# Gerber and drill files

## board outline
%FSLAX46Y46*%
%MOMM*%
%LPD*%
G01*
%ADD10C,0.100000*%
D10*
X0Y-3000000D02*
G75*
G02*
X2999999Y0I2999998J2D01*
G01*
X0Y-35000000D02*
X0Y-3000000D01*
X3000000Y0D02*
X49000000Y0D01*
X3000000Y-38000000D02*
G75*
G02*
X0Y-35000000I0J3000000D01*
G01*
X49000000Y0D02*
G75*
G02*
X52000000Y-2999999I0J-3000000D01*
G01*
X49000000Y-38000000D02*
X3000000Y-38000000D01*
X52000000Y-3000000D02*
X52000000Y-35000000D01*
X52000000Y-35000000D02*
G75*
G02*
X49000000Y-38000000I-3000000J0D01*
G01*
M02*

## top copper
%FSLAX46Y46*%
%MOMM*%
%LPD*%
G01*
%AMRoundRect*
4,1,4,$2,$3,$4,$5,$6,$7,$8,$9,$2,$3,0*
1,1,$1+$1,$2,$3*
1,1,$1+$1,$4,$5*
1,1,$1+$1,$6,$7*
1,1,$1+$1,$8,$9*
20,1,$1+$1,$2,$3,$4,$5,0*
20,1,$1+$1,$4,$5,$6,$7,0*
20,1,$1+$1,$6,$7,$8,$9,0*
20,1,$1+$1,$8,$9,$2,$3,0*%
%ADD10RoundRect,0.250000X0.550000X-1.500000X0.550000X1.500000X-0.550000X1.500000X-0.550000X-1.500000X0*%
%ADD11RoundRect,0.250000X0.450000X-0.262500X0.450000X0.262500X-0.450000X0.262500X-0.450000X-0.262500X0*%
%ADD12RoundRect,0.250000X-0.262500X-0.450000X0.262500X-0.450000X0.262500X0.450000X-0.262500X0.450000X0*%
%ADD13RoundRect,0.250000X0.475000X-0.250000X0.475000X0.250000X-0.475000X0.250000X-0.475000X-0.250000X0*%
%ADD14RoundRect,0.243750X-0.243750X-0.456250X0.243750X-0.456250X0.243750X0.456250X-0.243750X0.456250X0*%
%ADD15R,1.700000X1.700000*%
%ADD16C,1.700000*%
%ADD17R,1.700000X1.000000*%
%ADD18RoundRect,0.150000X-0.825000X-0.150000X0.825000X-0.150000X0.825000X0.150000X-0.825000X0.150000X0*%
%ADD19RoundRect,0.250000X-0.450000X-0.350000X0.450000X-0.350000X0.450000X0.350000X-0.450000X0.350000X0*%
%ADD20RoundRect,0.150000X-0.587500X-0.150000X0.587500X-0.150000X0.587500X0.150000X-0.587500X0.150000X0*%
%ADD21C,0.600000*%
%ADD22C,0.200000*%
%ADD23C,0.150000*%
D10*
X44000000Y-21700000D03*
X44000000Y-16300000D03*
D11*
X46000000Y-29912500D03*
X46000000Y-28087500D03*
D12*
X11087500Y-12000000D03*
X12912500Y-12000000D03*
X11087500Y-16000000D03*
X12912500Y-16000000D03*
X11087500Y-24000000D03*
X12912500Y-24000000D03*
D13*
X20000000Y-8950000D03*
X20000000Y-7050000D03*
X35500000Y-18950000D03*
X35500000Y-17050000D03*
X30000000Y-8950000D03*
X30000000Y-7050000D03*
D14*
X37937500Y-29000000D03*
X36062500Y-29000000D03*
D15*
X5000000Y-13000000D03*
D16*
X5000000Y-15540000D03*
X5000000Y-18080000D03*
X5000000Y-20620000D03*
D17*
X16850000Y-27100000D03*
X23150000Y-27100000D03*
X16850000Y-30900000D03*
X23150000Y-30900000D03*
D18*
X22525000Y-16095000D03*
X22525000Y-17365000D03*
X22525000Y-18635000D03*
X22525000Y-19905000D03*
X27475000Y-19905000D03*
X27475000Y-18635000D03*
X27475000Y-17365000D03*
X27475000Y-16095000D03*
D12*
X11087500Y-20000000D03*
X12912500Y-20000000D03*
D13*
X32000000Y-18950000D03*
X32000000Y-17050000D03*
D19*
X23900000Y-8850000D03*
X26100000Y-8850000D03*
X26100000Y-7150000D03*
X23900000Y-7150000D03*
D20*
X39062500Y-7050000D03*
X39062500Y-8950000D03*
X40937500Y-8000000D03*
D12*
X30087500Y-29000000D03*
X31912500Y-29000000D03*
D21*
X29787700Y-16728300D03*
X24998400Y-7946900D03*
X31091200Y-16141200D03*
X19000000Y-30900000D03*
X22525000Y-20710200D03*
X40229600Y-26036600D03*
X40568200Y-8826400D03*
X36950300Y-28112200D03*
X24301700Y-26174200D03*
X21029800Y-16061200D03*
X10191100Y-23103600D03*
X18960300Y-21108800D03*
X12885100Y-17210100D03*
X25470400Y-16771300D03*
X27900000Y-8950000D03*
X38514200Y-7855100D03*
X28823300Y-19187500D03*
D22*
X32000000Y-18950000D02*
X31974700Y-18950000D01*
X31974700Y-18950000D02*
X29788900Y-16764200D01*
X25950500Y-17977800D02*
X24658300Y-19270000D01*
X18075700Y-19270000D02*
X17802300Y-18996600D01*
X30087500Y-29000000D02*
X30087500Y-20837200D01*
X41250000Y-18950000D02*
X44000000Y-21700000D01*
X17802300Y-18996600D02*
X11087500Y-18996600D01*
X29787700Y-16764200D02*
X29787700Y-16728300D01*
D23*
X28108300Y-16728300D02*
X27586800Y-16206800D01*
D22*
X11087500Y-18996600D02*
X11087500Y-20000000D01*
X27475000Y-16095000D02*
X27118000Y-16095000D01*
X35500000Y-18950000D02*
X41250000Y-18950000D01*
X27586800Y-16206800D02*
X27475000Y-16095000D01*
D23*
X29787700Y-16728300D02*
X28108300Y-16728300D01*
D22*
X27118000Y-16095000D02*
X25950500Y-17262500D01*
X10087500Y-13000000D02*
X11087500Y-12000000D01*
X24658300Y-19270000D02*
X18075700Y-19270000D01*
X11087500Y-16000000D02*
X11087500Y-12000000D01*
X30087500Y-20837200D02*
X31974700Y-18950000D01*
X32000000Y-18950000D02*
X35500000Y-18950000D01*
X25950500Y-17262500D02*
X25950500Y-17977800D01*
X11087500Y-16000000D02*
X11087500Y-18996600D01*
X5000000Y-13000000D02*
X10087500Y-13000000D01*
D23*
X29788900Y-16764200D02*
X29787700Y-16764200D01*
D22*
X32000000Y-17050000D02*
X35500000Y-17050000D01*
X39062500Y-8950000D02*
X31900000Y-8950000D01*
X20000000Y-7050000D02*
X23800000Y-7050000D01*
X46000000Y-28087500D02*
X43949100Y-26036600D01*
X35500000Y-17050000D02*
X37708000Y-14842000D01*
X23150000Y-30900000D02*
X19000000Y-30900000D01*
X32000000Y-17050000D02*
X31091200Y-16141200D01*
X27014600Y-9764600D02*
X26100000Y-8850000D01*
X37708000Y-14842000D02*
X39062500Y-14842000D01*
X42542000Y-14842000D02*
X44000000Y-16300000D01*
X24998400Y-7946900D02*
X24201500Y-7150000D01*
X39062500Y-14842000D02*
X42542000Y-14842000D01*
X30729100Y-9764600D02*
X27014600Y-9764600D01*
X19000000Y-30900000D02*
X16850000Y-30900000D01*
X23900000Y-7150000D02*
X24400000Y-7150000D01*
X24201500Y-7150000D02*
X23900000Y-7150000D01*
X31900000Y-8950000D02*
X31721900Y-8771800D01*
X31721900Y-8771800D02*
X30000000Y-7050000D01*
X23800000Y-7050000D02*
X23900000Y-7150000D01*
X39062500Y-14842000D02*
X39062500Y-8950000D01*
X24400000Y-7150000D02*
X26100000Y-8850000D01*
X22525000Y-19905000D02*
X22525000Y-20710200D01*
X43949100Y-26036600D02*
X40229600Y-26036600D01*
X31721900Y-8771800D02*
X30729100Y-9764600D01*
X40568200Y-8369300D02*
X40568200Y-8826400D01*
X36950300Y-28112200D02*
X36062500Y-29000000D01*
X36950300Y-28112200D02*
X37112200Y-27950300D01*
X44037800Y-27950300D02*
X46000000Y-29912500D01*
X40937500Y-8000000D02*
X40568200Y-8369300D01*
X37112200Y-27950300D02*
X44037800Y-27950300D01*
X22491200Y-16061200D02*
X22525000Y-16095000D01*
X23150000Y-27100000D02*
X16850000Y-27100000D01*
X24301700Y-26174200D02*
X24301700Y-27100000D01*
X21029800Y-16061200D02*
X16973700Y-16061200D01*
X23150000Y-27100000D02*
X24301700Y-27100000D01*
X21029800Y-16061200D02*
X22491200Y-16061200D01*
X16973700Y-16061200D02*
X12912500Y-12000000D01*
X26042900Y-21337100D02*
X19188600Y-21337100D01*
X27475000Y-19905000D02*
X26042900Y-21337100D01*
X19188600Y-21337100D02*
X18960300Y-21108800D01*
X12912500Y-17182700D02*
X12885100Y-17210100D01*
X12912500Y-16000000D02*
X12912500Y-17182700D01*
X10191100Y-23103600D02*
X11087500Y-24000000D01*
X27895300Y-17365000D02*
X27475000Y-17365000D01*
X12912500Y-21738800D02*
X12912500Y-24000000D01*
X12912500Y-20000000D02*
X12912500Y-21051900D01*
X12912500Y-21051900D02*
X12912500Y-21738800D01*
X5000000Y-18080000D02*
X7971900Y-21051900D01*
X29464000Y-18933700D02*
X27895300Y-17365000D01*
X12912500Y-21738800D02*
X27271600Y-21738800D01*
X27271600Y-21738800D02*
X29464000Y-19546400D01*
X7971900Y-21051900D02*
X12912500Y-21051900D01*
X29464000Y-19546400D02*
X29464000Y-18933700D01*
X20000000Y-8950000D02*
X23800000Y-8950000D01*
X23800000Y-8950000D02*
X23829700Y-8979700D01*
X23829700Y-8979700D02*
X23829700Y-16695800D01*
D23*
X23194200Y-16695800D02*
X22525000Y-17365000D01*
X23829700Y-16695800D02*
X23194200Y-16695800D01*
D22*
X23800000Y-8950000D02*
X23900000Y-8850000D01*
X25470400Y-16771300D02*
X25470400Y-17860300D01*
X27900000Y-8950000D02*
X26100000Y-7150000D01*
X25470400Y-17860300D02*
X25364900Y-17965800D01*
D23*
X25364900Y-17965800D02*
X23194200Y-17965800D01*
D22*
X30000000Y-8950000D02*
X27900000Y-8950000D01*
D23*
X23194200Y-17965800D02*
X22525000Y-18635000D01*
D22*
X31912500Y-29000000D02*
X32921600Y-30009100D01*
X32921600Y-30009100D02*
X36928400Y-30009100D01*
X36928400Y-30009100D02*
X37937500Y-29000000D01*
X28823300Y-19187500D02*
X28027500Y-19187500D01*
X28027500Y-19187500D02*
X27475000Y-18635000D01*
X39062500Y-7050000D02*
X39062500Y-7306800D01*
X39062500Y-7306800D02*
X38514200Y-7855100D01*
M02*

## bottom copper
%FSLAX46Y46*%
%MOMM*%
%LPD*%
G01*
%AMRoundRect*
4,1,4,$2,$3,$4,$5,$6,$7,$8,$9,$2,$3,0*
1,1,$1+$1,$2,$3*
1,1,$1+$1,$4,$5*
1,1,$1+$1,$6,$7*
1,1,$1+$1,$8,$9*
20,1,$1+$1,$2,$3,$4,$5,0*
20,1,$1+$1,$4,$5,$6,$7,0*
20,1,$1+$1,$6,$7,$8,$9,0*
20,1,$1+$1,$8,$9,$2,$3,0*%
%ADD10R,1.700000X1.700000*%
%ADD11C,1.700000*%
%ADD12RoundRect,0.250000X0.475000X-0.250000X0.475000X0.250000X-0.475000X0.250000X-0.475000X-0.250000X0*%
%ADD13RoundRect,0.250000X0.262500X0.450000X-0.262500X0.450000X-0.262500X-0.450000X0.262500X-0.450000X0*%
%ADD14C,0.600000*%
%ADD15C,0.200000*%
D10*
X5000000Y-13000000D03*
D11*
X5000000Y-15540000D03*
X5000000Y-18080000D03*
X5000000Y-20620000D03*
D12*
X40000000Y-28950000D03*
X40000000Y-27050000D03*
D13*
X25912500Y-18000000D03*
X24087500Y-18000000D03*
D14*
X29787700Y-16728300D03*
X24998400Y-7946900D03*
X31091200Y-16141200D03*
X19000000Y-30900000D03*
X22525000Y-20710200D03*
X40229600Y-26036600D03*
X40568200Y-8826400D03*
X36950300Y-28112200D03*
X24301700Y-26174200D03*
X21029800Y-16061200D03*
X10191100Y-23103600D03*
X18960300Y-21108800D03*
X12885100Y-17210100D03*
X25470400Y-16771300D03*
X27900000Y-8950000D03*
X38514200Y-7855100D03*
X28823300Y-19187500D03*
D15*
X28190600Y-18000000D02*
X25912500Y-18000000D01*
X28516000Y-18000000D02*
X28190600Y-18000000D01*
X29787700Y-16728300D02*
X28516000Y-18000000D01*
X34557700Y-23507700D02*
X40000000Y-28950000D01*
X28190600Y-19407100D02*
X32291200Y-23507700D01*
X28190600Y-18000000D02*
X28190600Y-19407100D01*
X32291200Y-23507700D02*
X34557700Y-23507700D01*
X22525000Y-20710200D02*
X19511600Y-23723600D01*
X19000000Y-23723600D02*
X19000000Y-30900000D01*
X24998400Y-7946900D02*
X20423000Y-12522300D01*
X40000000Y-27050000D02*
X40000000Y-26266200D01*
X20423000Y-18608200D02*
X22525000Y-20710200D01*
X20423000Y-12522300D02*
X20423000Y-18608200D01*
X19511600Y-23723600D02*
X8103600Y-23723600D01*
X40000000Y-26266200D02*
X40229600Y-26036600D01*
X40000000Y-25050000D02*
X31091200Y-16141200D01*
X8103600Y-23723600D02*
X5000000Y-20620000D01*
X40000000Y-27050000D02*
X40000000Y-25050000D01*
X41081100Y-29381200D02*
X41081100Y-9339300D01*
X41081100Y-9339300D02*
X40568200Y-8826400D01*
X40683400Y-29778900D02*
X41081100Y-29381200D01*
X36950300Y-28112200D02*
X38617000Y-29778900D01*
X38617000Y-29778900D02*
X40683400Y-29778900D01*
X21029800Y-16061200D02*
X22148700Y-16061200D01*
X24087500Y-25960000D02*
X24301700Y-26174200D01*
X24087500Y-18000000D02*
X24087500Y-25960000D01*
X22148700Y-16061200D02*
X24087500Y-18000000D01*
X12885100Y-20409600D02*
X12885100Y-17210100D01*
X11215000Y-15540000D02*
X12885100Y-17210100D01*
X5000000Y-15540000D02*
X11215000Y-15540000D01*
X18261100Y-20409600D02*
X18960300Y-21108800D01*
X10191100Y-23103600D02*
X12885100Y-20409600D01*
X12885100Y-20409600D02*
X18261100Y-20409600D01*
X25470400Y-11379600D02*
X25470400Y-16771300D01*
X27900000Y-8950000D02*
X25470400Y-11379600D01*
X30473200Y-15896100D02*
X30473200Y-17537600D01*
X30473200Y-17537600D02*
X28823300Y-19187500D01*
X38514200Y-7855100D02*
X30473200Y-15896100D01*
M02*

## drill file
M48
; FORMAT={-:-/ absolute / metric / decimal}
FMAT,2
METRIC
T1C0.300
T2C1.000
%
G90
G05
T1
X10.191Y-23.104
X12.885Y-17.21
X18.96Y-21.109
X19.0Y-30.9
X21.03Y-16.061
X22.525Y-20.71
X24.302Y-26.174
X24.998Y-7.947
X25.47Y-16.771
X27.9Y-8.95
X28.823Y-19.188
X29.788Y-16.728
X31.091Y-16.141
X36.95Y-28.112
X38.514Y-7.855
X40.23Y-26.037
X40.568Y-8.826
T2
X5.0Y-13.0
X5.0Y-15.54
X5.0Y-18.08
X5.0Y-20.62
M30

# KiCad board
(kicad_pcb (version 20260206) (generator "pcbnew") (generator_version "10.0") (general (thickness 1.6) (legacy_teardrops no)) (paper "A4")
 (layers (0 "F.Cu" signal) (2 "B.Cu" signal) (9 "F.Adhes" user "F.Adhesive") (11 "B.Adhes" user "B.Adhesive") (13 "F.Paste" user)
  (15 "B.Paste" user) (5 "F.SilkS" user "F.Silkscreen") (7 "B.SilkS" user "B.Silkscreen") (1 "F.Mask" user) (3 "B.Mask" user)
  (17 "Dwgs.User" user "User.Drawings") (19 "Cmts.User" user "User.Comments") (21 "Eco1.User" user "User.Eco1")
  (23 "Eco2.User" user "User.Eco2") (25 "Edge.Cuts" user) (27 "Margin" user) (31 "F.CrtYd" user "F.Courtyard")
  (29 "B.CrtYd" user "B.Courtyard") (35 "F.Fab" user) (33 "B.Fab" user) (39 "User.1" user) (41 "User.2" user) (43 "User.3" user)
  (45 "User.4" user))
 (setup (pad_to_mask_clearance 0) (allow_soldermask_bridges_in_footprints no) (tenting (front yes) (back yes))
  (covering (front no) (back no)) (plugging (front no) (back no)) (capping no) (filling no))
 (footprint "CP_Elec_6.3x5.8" (layer "F.Cu") (at 44 19 90)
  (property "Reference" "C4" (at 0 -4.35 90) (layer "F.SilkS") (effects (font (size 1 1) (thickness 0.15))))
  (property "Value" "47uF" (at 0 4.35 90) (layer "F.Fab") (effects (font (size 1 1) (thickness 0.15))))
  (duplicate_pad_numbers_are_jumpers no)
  (pad "1" smd roundrect (at -2.7 0 90) (size 3.5 1.6) (layers "F.Cu" "F.Mask" "F.Paste") (roundrect_rratio 0.15625) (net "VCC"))
  (pad "2" smd roundrect (at 2.7 0 90) (size 3.5 1.6) (layers "F.Cu" "F.Mask" "F.Paste") (roundrect_rratio 0.15625) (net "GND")))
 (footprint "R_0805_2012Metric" (layer "F.Cu") (at 46 29 90)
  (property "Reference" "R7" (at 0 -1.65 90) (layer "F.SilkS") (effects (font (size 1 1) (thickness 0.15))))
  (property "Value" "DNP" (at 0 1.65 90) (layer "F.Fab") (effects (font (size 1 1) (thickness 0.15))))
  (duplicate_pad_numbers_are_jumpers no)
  (pad "1" smd roundrect (at -0.9125 0 90) (size 1.025 1.4) (layers "F.Cu" "F.Mask" "F.Paste") (roundrect_rratio 0.243902) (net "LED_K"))
  (pad "2" smd roundrect (at 0.9125 0 90) (size 1.025 1.4) (layers "F.Cu" "F.Mask" "F.Paste") (roundrect_rratio 0.243902) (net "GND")))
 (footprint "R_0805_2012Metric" (layer "F.Cu") (at 12 12)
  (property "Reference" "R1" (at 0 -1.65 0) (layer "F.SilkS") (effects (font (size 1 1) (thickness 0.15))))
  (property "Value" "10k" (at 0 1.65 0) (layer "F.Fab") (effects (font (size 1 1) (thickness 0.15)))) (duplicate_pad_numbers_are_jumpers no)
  (pad "1" smd roundrect (at -0.9125 0) (size 1.025 1.4) (layers "F.Cu" "F.Mask" "F.Paste") (roundrect_rratio 0.243902) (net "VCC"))
  (pad "2" smd roundrect (at 0.9125 0) (size 1.025 1.4) (layers "F.Cu" "F.Mask" "F.Paste") (roundrect_rratio 0.243902) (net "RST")))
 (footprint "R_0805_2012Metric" (layer "F.Cu") (at 12 16)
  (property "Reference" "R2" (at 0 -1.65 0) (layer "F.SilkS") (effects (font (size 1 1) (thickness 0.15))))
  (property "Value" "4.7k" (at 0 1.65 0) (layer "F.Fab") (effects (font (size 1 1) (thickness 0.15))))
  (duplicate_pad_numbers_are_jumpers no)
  (pad "1" smd roundrect (at -0.9125 0) (size 1.025 1.4) (layers "F.Cu" "F.Mask" "F.Paste") (roundrect_rratio 0.243902) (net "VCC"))
  (pad "2" smd roundrect (at 0.9125 0) (size 1.025 1.4) (layers "F.Cu" "F.Mask" "F.Paste") (roundrect_rratio 0.243902) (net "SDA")))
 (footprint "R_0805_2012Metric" (layer "F.Cu") (at 12 24)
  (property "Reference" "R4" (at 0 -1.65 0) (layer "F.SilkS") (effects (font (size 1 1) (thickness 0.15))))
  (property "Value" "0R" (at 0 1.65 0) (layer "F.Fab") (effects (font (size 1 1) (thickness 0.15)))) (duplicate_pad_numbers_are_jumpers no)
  (pad "1" smd roundrect (at -0.9125 0) (size 1.025 1.4) (layers "F.Cu" "F.Mask" "F.Paste") (roundrect_rratio 0.243902) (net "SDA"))
  (pad "2" smd roundrect (at 0.9125 0) (size 1.025 1.4) (layers "F.Cu" "F.Mask" "F.Paste") (roundrect_rratio 0.243902) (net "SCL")))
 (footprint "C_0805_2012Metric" (layer "F.Cu") (at 20 8 90)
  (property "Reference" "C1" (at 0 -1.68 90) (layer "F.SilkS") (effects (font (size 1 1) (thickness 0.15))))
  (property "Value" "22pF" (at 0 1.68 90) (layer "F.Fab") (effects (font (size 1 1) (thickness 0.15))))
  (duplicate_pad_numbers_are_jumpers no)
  (pad "1" smd roundrect (at -0.95 0 90) (size 1 1.45) (layers "F.Cu" "F.Mask" "F.Paste") (roundrect_rratio 0.25) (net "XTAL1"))
  (pad "2" smd roundrect (at 0.95 0 90) (size 1 1.45) (layers "F.Cu" "F.Mask" "F.Paste") (roundrect_rratio 0.25) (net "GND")))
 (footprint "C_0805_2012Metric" (layer "F.Cu") (at 35.5 18 90)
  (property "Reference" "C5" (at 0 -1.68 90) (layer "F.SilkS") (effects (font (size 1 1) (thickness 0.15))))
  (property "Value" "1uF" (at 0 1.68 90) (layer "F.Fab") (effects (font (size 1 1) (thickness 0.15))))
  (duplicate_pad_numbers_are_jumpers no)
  (pad "1" smd roundrect (at -0.95 0 90) (size 1 1.45) (layers "F.Cu" "F.Mask" "F.Paste") (roundrect_rratio 0.25) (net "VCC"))
  (pad "2" smd roundrect (at 0.95 0 90) (size 1 1.45) (layers "F.Cu" "F.Mask" "F.Paste") (roundrect_rratio 0.25) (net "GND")))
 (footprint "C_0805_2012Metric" (layer "F.Cu") (at 30 8 90)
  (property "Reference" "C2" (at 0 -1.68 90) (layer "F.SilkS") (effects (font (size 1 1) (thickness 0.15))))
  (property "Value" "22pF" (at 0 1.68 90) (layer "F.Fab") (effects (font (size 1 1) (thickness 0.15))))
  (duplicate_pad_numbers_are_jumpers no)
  (pad "1" smd roundrect (at -0.95 0 90) (size 1 1.45) (layers "F.Cu" "F.Mask" "F.Paste") (roundrect_rratio 0.25) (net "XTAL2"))
  (pad "2" smd roundrect (at 0.95 0 90) (size 1 1.45) (layers "F.Cu" "F.Mask" "F.Paste") (roundrect_rratio 0.25) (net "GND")))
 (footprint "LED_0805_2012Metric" (layer "F.Cu") (at 37 29)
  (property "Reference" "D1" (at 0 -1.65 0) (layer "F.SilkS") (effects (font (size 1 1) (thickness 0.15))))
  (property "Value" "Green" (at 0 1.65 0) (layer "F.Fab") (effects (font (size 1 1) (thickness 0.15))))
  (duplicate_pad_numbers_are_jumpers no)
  (pad "A" smd roundrect (at 0.9375 0) (size 0.975 1.4) (layers "F.Cu" "F.Mask" "F.Paste") (roundrect_rratio 0.25) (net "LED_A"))
  (pad "K" smd roundrect (at -0.9375 0) (size 0.975 1.4) (layers "F.Cu" "F.Mask" "F.Paste") (roundrect_rratio 0.25) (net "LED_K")))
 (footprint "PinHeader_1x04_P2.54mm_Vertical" (layer "F.Cu") (at 5 13)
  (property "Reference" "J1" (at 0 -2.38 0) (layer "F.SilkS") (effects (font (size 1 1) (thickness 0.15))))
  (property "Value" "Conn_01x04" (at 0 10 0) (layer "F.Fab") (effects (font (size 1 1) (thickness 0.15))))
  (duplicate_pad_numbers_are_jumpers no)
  (pad "1" thru_hole rect (at 0 0) (size 1.7 1.7) (drill 1) (layers "*.Cu" "*.Mask") (remove_unused_layers no) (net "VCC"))
  (pad "2" thru_hole circle (at 0 2.54) (size 1.7 1.7) (drill 1) (layers "*.Cu" "*.Mask") (remove_unused_layers no) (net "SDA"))
  (pad "3" thru_hole circle (at 0 5.08) (size 1.7 1.7) (drill 1) (layers "*.Cu" "*.Mask") (remove_unused_layers no) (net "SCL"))
  (pad "4" thru_hole circle (at 0 7.62) (size 1.7 1.7) (drill 1) (layers "*.Cu" "*.Mask") (remove_unused_layers no) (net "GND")))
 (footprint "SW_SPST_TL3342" (layer "F.Cu") (at 20 29)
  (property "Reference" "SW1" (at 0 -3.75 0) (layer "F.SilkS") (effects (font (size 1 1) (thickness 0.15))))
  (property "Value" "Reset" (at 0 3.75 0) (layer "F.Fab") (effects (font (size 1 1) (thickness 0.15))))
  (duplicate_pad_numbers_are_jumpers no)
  (pad "1" smd rect (at -3.15 -1.9) (size 1.7 1) (layers "F.Cu" "F.Mask" "F.Paste") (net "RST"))
  (pad "1" smd rect (at 3.15 -1.9) (size 1.7 1) (layers "F.Cu" "F.Mask" "F.Paste") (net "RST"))
  (pad "2" smd rect (at -3.15 1.9) (size 1.7 1) (layers "F.Cu" "F.Mask" "F.Paste") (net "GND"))
  (pad "2" smd rect (at 3.15 1.9) (size 1.7 1) (layers "F.Cu" "F.Mask" "F.Paste") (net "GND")))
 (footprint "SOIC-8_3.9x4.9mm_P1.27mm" (layer "F.Cu") (at 25 18)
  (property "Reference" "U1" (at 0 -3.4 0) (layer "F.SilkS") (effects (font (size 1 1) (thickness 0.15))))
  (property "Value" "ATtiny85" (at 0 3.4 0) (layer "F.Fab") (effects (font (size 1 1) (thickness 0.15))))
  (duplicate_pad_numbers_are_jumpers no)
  (pad "1" smd roundrect (at -2.475 -1.905) (size 1.95 0.6) (layers "F.Cu" "F.Mask" "F.Paste") (roundrect_rratio 0.25) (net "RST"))
  (pad "2" smd roundrect (at -2.475 -0.635) (size 1.95 0.6) (layers "F.Cu" "F.Mask" "F.Paste") (roundrect_rratio 0.25) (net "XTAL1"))
  (pad "3" smd roundrect (at -2.475 0.635) (size 1.95 0.6) (layers "F.Cu" "F.Mask" "F.Paste") (roundrect_rratio 0.25) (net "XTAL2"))
  (pad "4" smd roundrect (at -2.475 1.905) (size 1.95 0.6) (layers "F.Cu" "F.Mask" "F.Paste") (roundrect_rratio 0.25) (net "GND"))
  (pad "5" smd roundrect (at 2.475 1.905) (size 1.95 0.6) (layers "F.Cu" "F.Mask" "F.Paste") (roundrect_rratio 0.25) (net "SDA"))
  (pad "6" smd roundrect (at 2.475 0.635) (size 1.95 0.6) (layers "F.Cu" "F.Mask" "F.Paste") (roundrect_rratio 0.25) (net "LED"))
  (pad "7" smd roundrect (at 2.475 -0.635) (size 1.95 0.6) (layers "F.Cu" "F.Mask" "F.Paste") (roundrect_rratio 0.25) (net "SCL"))
  (pad "8" smd roundrect (at 2.475 -1.905) (size 1.95 0.6) (layers "F.Cu" "F.Mask" "F.Paste") (roundrect_rratio 0.25) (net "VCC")))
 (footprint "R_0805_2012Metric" (layer "F.Cu") (at 12 20)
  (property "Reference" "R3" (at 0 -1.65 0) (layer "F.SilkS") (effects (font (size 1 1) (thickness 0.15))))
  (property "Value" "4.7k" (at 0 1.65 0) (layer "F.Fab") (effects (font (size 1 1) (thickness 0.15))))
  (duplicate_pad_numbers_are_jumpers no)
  (pad "1" smd roundrect (at -0.9125 0) (size 1.025 1.4) (layers "F.Cu" "F.Mask" "F.Paste") (roundrect_rratio 0.243902) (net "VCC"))
  (pad "2" smd roundrect (at 0.9125 0) (size 1.025 1.4) (layers "F.Cu" "F.Mask" "F.Paste") (roundrect_rratio 0.243902) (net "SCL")))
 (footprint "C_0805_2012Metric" (layer "F.Cu") (at 32 18 90)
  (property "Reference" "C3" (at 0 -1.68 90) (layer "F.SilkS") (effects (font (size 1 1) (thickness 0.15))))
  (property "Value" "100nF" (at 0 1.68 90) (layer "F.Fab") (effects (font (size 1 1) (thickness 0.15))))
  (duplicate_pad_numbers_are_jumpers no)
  (pad "1" smd roundrect (at -0.95 0 90) (size 1 1.45) (layers "F.Cu" "F.Mask" "F.Paste") (roundrect_rratio 0.25) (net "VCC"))
  (pad "2" smd roundrect (at 0.95 0 90) (size 1 1.45) (layers "F.Cu" "F.Mask" "F.Paste") (roundrect_rratio 0.25) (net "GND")))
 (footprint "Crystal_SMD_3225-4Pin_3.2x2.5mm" (layer "F.Cu") (at 25 8)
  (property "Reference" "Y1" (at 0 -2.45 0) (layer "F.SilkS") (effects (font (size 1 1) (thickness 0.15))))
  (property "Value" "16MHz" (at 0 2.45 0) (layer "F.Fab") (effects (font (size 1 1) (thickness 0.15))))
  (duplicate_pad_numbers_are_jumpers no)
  (pad "1" smd roundrect (at -1.1 0.85) (size 1.4 1.2) (layers "F.Cu" "F.Mask" "F.Paste") (roundrect_rratio 0.208333) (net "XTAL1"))
  (pad "2" smd roundrect (at 1.1 0.85) (size 1.4 1.2) (layers "F.Cu" "F.Mask" "F.Paste") (roundrect_rratio 0.208333) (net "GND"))
  (pad "3" smd roundrect (at 1.1 -0.85) (size 1.4 1.2) (layers "F.Cu" "F.Mask" "F.Paste") (roundrect_rratio 0.208333) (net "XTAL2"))
  (pad "4" smd roundrect (at -1.1 -0.85) (size 1.4 1.2) (layers "F.Cu" "F.Mask" "F.Paste") (roundrect_rratio 0.208333) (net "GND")))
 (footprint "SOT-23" (layer "F.Cu") (at 40 8)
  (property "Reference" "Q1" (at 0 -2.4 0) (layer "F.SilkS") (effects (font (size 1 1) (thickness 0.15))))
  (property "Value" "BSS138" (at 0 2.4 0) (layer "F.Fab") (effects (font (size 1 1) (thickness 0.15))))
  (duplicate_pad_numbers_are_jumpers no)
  (pad "1" smd roundrect (at -0.9375 -0.95) (size 1.475 0.6) (layers "F.Cu" "F.Mask" "F.Paste") (roundrect_rratio 0.25) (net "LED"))
  (pad "2" smd roundrect (at -0.9375 0.95) (size 1.475 0.6) (layers "F.Cu" "F.Mask" "F.Paste") (roundrect_rratio 0.25) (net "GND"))
  (pad "3" smd roundrect (at 0.9375 0) (size 1.475 0.6) (layers "F.Cu" "F.Mask" "F.Paste") (roundrect_rratio 0.25) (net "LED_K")))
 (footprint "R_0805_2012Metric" (layer "F.Cu") (at 31 29)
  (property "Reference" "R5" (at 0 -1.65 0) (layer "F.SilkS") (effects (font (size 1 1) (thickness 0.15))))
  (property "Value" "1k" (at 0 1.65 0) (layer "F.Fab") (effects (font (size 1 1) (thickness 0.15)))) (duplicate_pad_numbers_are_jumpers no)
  (pad "1" smd roundrect (at -0.9125 0) (size 1.025 1.4) (layers "F.Cu" "F.Mask" "F.Paste") (roundrect_rratio 0.243902) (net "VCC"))
  (pad "2" smd roundrect (at 0.9125 0) (size 1.025 1.4) (layers "F.Cu" "F.Mask" "F.Paste") (roundrect_rratio 0.243902) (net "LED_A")))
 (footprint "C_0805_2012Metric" (layer "B.Cu") (at 40 28 90)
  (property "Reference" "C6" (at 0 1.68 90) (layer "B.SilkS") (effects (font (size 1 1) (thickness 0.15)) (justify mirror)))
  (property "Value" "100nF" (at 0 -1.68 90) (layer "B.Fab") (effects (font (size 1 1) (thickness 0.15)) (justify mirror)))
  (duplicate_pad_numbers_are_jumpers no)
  (pad "1" smd roundrect (at -0.95 0 90) (size 1 1.45) (layers "B.Cu" "B.Mask" "B.Paste") (roundrect_rratio 0.25) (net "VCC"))
  (pad "2" smd roundrect (at 0.95 0 90) (size 1 1.45) (layers "B.Cu" "B.Mask" "B.Paste") (roundrect_rratio 0.25) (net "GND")))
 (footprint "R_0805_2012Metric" (layer "B.Cu") (at 25 18 180)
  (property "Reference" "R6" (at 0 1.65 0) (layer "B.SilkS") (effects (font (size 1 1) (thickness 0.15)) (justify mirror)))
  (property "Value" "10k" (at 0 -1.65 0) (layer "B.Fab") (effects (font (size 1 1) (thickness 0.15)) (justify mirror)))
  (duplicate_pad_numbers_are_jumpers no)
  (pad "1" smd roundrect (at -0.9125 0 180) (size 1.025 1.4) (layers "B.Cu" "B.Mask" "B.Paste") (roundrect_rratio 0.243902) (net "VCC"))
  (pad "2" smd roundrect (at 0.9125 0 180) (size 1.025 1.4) (layers "B.Cu" "B.Mask" "B.Paste") (roundrect_rratio 0.243902) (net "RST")))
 (gr_arc (start 0 3) (mid 0.878679 0.878679) (end 2.999999 0) (stroke (width 0.1) (type default)) (layer "Edge.Cuts"))
 (gr_line (start 0 35) (end 0 3) (stroke (width 0.1) (type default)) (layer "Edge.Cuts"))
 (gr_line (start 3 0) (end 49 0) (stroke (width 0.1) (type default)) (layer "Edge.Cuts"))
 (gr_arc (start 3 38) (mid 0.878679 37.12132) (end 0 35) (stroke (width 0.1) (type default)) (layer "Edge.Cuts"))
 (gr_arc (start 49 0) (mid 51.12132 0.878679) (end 52 2.999999) (stroke (width 0.1) (type default)) (layer "Edge.Cuts"))
 (gr_line (start 49 38) (end 3 38) (stroke (width 0.1) (type default)) (layer "Edge.Cuts"))
 (gr_line (start 52 3) (end 52 35) (stroke (width 0.1) (type default)) (layer "Edge.Cuts"))
 (gr_arc (start 52 35) (mid 51.12132 37.12132) (end 49 38) (stroke (width 0.1) (type default)) (layer "Edge.Cuts"))
 (segment (start 32 18.95) (end 31.9747 18.95) (width 0.2) (layer "F.Cu") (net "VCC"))
 (segment (start 31.9747 18.95) (end 29.7889 16.7642) (width 0.2) (layer "F.Cu") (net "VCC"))
 (segment (start 25.9505 17.9778) (end 24.6583 19.27) (width 0.2) (layer "F.Cu") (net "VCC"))
 (segment (start 18.0757 19.27) (end 17.8023 18.9966) (width 0.2) (layer "F.Cu") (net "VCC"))
 (segment (start 30.0875 29) (end 30.0875 20.8372) (width 0.2) (layer "F.Cu") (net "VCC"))
 (segment (start 41.25 18.95) (end 44 21.7) (width 0.2) (layer "F.Cu") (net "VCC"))
 (segment (start 17.8023 18.9966) (end 11.0875 18.9966) (width 0.2) (layer "F.Cu") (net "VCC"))
 (segment (start 29.7877 16.7642) (end 29.7877 16.7283) (width 0.2) (layer "F.Cu") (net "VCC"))
 (segment (start 28.1083 16.7283) (end 27.5868 16.2068) (width 0.15) (layer "F.Cu") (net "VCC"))
 (segment (start 11.0875 18.9966) (end 11.0875 20) (width 0.2) (layer "F.Cu") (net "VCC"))
 (segment (start 27.475 16.095) (end 27.118 16.095) (width 0.2) (layer "F.Cu") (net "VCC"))
 (segment (start 35.5 18.95) (end 41.25 18.95) (width 0.2) (layer "F.Cu") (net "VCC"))
 (segment (start 27.5868 16.2068) (end 27.475 16.095) (width 0.2) (layer "F.Cu") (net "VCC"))
 (segment (start 29.7877 16.7283) (end 28.1083 16.7283) (width 0.15) (layer "F.Cu") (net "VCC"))
 (segment (start 27.118 16.095) (end 25.9505 17.2625) (width 0.2) (layer "F.Cu") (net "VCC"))
 (segment (start 10.0875 13) (end 11.0875 12) (width 0.2) (layer "F.Cu") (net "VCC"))
 (segment (start 24.6583 19.27) (end 18.0757 19.27) (width 0.2) (layer "F.Cu") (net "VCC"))
 (segment (start 11.0875 16) (end 11.0875 12) (width 0.2) (layer "F.Cu") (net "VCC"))
 (segment (start 30.0875 20.8372) (end 31.9747 18.95) (width 0.2) (layer "F.Cu") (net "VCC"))
 (segment (start 32 18.95) (end 35.5 18.95) (width 0.2) (layer "F.Cu") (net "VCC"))
 (segment (start 25.9505 17.2625) (end 25.9505 17.9778) (width 0.2) (layer "F.Cu") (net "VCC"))
 (segment (start 11.0875 16) (end 11.0875 18.9966) (width 0.2) (layer "F.Cu") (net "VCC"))
 (segment (start 5 13) (end 10.0875 13) (width 0.2) (layer "F.Cu") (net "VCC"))
 (segment (start 29.7889 16.7642) (end 29.7877 16.7642) (width 0.15) (layer "F.Cu") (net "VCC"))
 (via (at 29.7877 16.7283) (size 0.6) (drill 0.3) (layers "F.Cu" "B.Cu") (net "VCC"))
 (segment (start 28.1906 18) (end 25.9125 18) (width 0.2) (layer "B.Cu") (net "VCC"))
 (segment (start 28.516 18) (end 28.1906 18) (width 0.2) (layer "B.Cu") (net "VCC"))
 (segment (start 29.7877 16.7283) (end 28.516 18) (width 0.2) (layer "B.Cu") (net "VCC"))
 (segment (start 34.5577 23.5077) (end 40 28.95) (width 0.2) (layer "B.Cu") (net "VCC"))
 (segment (start 28.1906 19.4071) (end 32.2912 23.5077) (width 0.2) (layer "B.Cu") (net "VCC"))
 (segment (start 28.1906 18) (end 28.1906 19.4071) (width 0.2) (layer "B.Cu") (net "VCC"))
 (segment (start 32.2912 23.5077) (end 34.5577 23.5077) (width 0.2) (layer "B.Cu") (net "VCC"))
 (segment (start 32 17.05) (end 35.5 17.05) (width 0.2) (layer "F.Cu") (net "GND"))
 (segment (start 39.0625 8.95) (end 31.9 8.95) (width 0.2) (layer "F.Cu") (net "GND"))
 (segment (start 20 7.05) (end 23.8 7.05) (width 0.2) (layer "F.Cu") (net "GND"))
 (segment (start 46 28.0875) (end 43.9491 26.0366) (width 0.2) (layer "F.Cu") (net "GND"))
 (segment (start 35.5 17.05) (end 37.708 14.842) (width 0.2) (layer "F.Cu") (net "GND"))
 (segment (start 23.15 30.9) (end 19 30.9) (width 0.2) (layer "F.Cu") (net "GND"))
 (segment (start 32 17.05) (end 31.0912 16.1412) (width 0.2) (layer "F.Cu") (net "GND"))
 (segment (start 27.0146 9.7646) (end 26.1 8.85) (width 0.2) (layer "F.Cu") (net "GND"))
 (segment (start 37.708 14.842) (end 39.0625 14.842) (width 0.2) (layer "F.Cu") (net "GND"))
 (segment (start 42.542 14.842) (end 44 16.3) (width 0.2) (layer "F.Cu") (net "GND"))
 (segment (start 24.9984 7.9469) (end 24.2015 7.15) (width 0.2) (layer "F.Cu") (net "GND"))
 (segment (start 39.0625 14.842) (end 42.542 14.842) (width 0.2) (layer "F.Cu") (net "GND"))
 (segment (start 30.7291 9.7646) (end 27.0146 9.7646) (width 0.2) (layer "F.Cu") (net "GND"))
 (segment (start 19 30.9) (end 16.85 30.9) (width 0.2) (layer "F.Cu") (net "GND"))
 (segment (start 23.9 7.15) (end 24.4 7.15) (width 0.2) (layer "F.Cu") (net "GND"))
 (segment (start 24.2015 7.15) (end 23.9 7.15) (width 0.2) (layer "F.Cu") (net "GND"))
 (segment (start 31.9 8.95) (end 31.7219 8.7718) (width 0.2) (layer "F.Cu") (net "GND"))
 (segment (start 31.7219 8.7718) (end 30 7.05) (width 0.2) (layer "F.Cu") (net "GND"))
 (segment (start 23.8 7.05) (end 23.9 7.15) (width 0.2) (layer "F.Cu") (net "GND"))
 (segment (start 39.0625 14.842) (end 39.0625 8.95) (width 0.2) (layer "F.Cu") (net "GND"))
 (segment (start 24.4 7.15) (end 26.1 8.85) (width 0.2) (layer "F.Cu") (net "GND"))
 (segment (start 22.525 19.905) (end 22.525 20.7102) (width 0.2) (layer "F.Cu") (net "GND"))
 (segment (start 43.9491 26.0366) (end 40.2296 26.0366) (width 0.2) (layer "F.Cu") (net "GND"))
 (segment (start 31.7219 8.7718) (end 30.7291 9.7646) (width 0.2) (layer "F.Cu") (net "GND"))
 (via (at 24.9984 7.9469) (size 0.6) (drill 0.3) (layers "F.Cu" "B.Cu") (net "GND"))
 (via (at 31.0912 16.1412) (size 0.6) (drill 0.3) (layers "F.Cu" "B.Cu") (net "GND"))
 (via (at 19 30.9) (size 0.6) (drill 0.3) (layers "F.Cu" "B.Cu") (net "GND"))
 (via (at 22.525 20.7102) (size 0.6) (drill 0.3) (layers "F.Cu" "B.Cu") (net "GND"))
 (via (at 40.2296 26.0366) (size 0.6) (drill 0.3) (layers "F.Cu" "B.Cu") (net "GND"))
 (segment (start 22.525 20.7102) (end 19.5116 23.7236) (width 0.2) (layer "B.Cu") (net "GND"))
 (segment (start 19 23.7236) (end 19 30.9) (width 0.2) (layer "B.Cu") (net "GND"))
 (segment (start 24.9984 7.9469) (end 20.423 12.5223) (width 0.2) (layer "B.Cu") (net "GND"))
 (segment (start 40 27.05) (end 40 26.2662) (width 0.2) (layer "B.Cu") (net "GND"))
 (segment (start 20.423 18.6082) (end 22.525 20.7102) (width 0.2) (layer "B.Cu") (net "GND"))
 (segment (start 20.423 12.5223) (end 20.423 18.6082) (width 0.2) (layer "B.Cu") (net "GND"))
 (segment (start 19.5116 23.7236) (end 8.1036 23.7236) (width 0.2) (layer "B.Cu") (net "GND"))
 (segment (start 40 26.2662) (end 40.2296 26.0366) (width 0.2) (layer "B.Cu") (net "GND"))
 (segment (start 40 25.05) (end 31.0912 16.1412) (width 0.2) (layer "B.Cu") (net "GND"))
 (segment (start 8.1036 23.7236) (end 5 20.62) (width 0.2) (layer "B.Cu") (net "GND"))
 (segment (start 40 27.05) (end 40 25.05) (width 0.2) (layer "B.Cu") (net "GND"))
 (segment (start 40.5682 8.3693) (end 40.5682 8.8264) (width 0.2) (layer "F.Cu") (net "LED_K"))
 (segment (start 36.9503 28.1122) (end 36.0625 29) (width 0.2) (layer "F.Cu") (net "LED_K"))
 (segment (start 36.9503 28.1122) (end 37.1122 27.9503) (width 0.2) (layer "F.Cu") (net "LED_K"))
 (segment (start 44.0378 27.9503) (end 46 29.9125) (width 0.2) (layer "F.Cu") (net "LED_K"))
 (segment (start 40.9375 8) (end 40.5682 8.3693) (width 0.2) (layer "F.Cu") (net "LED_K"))
 (segment (start 37.1122 27.9503) (end 44.0378 27.9503) (width 0.2) (layer "F.Cu") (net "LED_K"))
 (via (at 40.5682 8.8264) (size 0.6) (drill 0.3) (layers "F.Cu" "B.Cu") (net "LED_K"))
 (via (at 36.9503 28.1122) (size 0.6) (drill 0.3) (layers "F.Cu" "B.Cu") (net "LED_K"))
 (segment (start 41.0811 29.3812) (end 41.0811 9.3393) (width 0.2) (layer "B.Cu") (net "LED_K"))
 (segment (start 41.0811 9.3393) (end 40.5682 8.8264) (width 0.2) (layer "B.Cu") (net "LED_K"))
 (segment (start 40.6834 29.7789) (end 41.0811 29.3812) (width 0.2) (layer "B.Cu") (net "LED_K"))
 (segment (start 36.9503 28.1122) (end 38.617 29.7789) (width 0.2) (layer "B.Cu") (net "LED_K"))
 (segment (start 38.617 29.7789) (end 40.6834 29.7789) (width 0.2) (layer "B.Cu") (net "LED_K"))
 (segment (start 22.4912 16.0612) (end 22.525 16.095) (width 0.2) (layer "F.Cu") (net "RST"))
 (segment (start 23.15 27.1) (end 16.85 27.1) (width 0.2) (layer "F.Cu") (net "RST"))
 (segment (start 24.3017 26.1742) (end 24.3017 27.1) (width 0.2) (layer "F.Cu") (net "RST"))
 (segment (start 21.0298 16.0612) (end 16.9737 16.0612) (width 0.2) (layer "F.Cu") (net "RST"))
 (segment (start 23.15 27.1) (end 24.3017 27.1) (width 0.2) (layer "F.Cu") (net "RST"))
 (segment (start 21.0298 16.0612) (end 22.4912 16.0612) (width 0.2) (layer "F.Cu") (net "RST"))
 (segment (start 16.9737 16.0612) (end 12.9125 12) (width 0.2) (layer "F.Cu") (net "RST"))
 (via (at 24.3017 26.1742) (size 0.6) (drill 0.3) (layers "F.Cu" "B.Cu") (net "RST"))
 (via (at 21.0298 16.0612) (size 0.6) (drill 0.3) (layers "F.Cu" "B.Cu") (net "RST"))
 (segment (start 21.0298 16.0612) (end 22.1487 16.0612) (width 0.2) (layer "B.Cu") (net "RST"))
 (segment (start 24.0875 25.96) (end 24.3017 26.1742) (width 0.2) (layer "B.Cu") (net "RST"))
 (segment (start 24.0875 18) (end 24.0875 25.96) (width 0.2) (layer "B.Cu") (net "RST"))
 (segment (start 22.1487 16.0612) (end 24.0875 18) (width 0.2) (layer "B.Cu") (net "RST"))
 (segment (start 26.0429 21.3371) (end 19.1886 21.3371) (width 0.2) (layer "F.Cu") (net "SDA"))
 (segment (start 27.475 19.905) (end 26.0429 21.3371) (width 0.2) (layer "F.Cu") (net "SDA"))
 (segment (start 19.1886 21.3371) (end 18.9603 21.1088) (width 0.2) (layer "F.Cu") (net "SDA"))
 (segment (start 12.9125 17.1827) (end 12.8851 17.2101) (width 0.2) (layer "F.Cu") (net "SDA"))
 (segment (start 12.9125 16) (end 12.9125 17.1827) (width 0.2) (layer "F.Cu") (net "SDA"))
 (segment (start 10.1911 23.1036) (end 11.0875 24) (width 0.2) (layer "F.Cu") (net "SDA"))
 (via (at 10.1911 23.1036) (size 0.6) (drill 0.3) (layers "F.Cu" "B.Cu") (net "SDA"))
 (via (at 18.9603 21.1088) (size 0.6) (drill 0.3) (layers "F.Cu" "B.Cu") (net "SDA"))
 (via (at 12.8851 17.2101) (size 0.6) (drill 0.3) (layers "F.Cu" "B.Cu") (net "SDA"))
 (segment (start 12.8851 20.4096) (end 12.8851 17.2101) (width 0.2) (layer "B.Cu") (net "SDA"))
 (segment (start 11.215 15.54) (end 12.8851 17.2101) (width 0.2) (layer "B.Cu") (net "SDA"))
 (segment (start 5 15.54) (end 11.215 15.54) (width 0.2) (layer "B.Cu") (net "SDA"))
 (segment (start 18.2611 20.4096) (end 18.9603 21.1088) (width 0.2) (layer "B.Cu") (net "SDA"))
 (segment (start 10.1911 23.1036) (end 12.8851 20.4096) (width 0.2) (layer "B.Cu") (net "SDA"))
 (segment (start 12.8851 20.4096) (end 18.2611 20.4096) (width 0.2) (layer "B.Cu") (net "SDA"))
 (segment (start 27.8953 17.365) (end 27.475 17.365) (width 0.2) (layer "F.Cu") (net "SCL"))
 (segment (start 12.9125 21.7388) (end 12.9125 24) (width 0.2) (layer "F.Cu") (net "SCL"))
 (segment (start 12.9125 20) (end 12.9125 21.0519) (width 0.2) (layer "F.Cu") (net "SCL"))
 (segment (start 12.9125 21.0519) (end 12.9125 21.7388) (width 0.2) (layer "F.Cu") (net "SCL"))
 (segment (start 5 18.08) (end 7.9719 21.0519) (width 0.2) (layer "F.Cu") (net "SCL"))
 (segment (start 29.464 18.9337) (end 27.8953 17.365) (width 0.2) (layer "F.Cu") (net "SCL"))
 (segment (start 12.9125 21.7388) (end 27.2716 21.7388) (width 0.2) (layer "F.Cu") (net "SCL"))
 (segment (start 27.2716 21.7388) (end 29.464 19.5464) (width 0.2) (layer "F.Cu") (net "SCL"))
 (segment (start 7.9719 21.0519) (end 12.9125 21.0519) (width 0.2) (layer "F.Cu") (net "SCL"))
 (segment (start 29.464 19.5464) (end 29.464 18.9337) (width 0.2) (layer "F.Cu") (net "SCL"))
 (segment (start 20 8.95) (end 23.8 8.95) (width 0.2) (layer "F.Cu") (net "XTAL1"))
 (segment (start 23.8 8.95) (end 23.8297 8.9797) (width 0.2) (layer "F.Cu") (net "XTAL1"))
 (segment (start 23.8297 8.9797) (end 23.8297 16.6958) (width 0.2) (layer "F.Cu") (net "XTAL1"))
 (segment (start 23.1942 16.6958) (end 22.525 17.365) (width 0.15) (layer "F.Cu") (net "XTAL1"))
 (segment (start 23.8297 16.6958) (end 23.1942 16.6958) (width 0.15) (layer "F.Cu") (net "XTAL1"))
 (segment (start 23.8 8.95) (end 23.9 8.85) (width 0.2) (layer "F.Cu") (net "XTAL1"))
 (segment (start 25.4704 16.7713) (end 25.4704 17.8603) (width 0.2) (layer "F.Cu") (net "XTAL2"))
 (segment (start 27.9 8.95) (end 26.1 7.15) (width 0.2) (layer "F.Cu") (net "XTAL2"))
 (segment (start 25.4704 17.8603) (end 25.3649 17.9658) (width 0.2) (layer "F.Cu") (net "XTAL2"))
 (segment (start 25.3649 17.9658) (end 23.1942 17.9658) (width 0.15) (layer "F.Cu") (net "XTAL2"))
 (segment (start 30 8.95) (end 27.9 8.95) (width 0.2) (layer "F.Cu") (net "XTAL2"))
 (segment (start 23.1942 17.9658) (end 22.525 18.635) (width 0.15) (layer "F.Cu") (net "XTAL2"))
 (via (at 25.4704 16.7713) (size 0.6) (drill 0.3) (layers "F.Cu" "B.Cu") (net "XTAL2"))
 (via (at 27.9 8.95) (size 0.6) (drill 0.3) (layers "F.Cu" "B.Cu") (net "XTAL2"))
 (segment (start 25.4704 11.3796) (end 25.4704 16.7713) (width 0.2) (layer "B.Cu") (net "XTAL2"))
 (segment (start 27.9 8.95) (end 25.4704 11.3796) (width 0.2) (layer "B.Cu") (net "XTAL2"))
 (segment (start 31.9125 29) (end 32.9216 30.0091) (width 0.2) (layer "F.Cu") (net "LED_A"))
 (segment (start 32.9216 30.0091) (end 36.9284 30.0091) (width 0.2) (layer "F.Cu") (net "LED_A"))
 (segment (start 36.9284 30.0091) (end 37.9375 29) (width 0.2) (layer "F.Cu") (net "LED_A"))
 (segment (start 28.8233 19.1875) (end 28.0275 19.1875) (width 0.2) (layer "F.Cu") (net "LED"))
 (segment (start 28.0275 19.1875) (end 27.475 18.635) (width 0.2) (layer "F.Cu") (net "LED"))
 (segment (start 39.0625 7.05) (end 39.0625 7.3068) (width 0.2) (layer "F.Cu") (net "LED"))
 (segment (start 39.0625 7.3068) (end 38.5142 7.8551) (width 0.2) (layer "F.Cu") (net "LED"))
 (via (at 38.5142 7.8551) (size 0.6) (drill 0.3) (layers "F.Cu" "B.Cu") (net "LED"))
 (via (at 28.8233 19.1875) (size 0.6) (drill 0.3) (layers "F.Cu" "B.Cu") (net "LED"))
 (segment (start 30.4732 15.8961) (end 30.4732 17.5376) (width 0.2) (layer "B.Cu") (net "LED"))
 (segment (start 30.4732 17.5376) (end 28.8233 19.1875) (width 0.2) (layer "B.Cu") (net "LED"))
 (segment (start 38.5142 7.8551) (end 30.4732 15.8961) (width 0.2) (layer "B.Cu") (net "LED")))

